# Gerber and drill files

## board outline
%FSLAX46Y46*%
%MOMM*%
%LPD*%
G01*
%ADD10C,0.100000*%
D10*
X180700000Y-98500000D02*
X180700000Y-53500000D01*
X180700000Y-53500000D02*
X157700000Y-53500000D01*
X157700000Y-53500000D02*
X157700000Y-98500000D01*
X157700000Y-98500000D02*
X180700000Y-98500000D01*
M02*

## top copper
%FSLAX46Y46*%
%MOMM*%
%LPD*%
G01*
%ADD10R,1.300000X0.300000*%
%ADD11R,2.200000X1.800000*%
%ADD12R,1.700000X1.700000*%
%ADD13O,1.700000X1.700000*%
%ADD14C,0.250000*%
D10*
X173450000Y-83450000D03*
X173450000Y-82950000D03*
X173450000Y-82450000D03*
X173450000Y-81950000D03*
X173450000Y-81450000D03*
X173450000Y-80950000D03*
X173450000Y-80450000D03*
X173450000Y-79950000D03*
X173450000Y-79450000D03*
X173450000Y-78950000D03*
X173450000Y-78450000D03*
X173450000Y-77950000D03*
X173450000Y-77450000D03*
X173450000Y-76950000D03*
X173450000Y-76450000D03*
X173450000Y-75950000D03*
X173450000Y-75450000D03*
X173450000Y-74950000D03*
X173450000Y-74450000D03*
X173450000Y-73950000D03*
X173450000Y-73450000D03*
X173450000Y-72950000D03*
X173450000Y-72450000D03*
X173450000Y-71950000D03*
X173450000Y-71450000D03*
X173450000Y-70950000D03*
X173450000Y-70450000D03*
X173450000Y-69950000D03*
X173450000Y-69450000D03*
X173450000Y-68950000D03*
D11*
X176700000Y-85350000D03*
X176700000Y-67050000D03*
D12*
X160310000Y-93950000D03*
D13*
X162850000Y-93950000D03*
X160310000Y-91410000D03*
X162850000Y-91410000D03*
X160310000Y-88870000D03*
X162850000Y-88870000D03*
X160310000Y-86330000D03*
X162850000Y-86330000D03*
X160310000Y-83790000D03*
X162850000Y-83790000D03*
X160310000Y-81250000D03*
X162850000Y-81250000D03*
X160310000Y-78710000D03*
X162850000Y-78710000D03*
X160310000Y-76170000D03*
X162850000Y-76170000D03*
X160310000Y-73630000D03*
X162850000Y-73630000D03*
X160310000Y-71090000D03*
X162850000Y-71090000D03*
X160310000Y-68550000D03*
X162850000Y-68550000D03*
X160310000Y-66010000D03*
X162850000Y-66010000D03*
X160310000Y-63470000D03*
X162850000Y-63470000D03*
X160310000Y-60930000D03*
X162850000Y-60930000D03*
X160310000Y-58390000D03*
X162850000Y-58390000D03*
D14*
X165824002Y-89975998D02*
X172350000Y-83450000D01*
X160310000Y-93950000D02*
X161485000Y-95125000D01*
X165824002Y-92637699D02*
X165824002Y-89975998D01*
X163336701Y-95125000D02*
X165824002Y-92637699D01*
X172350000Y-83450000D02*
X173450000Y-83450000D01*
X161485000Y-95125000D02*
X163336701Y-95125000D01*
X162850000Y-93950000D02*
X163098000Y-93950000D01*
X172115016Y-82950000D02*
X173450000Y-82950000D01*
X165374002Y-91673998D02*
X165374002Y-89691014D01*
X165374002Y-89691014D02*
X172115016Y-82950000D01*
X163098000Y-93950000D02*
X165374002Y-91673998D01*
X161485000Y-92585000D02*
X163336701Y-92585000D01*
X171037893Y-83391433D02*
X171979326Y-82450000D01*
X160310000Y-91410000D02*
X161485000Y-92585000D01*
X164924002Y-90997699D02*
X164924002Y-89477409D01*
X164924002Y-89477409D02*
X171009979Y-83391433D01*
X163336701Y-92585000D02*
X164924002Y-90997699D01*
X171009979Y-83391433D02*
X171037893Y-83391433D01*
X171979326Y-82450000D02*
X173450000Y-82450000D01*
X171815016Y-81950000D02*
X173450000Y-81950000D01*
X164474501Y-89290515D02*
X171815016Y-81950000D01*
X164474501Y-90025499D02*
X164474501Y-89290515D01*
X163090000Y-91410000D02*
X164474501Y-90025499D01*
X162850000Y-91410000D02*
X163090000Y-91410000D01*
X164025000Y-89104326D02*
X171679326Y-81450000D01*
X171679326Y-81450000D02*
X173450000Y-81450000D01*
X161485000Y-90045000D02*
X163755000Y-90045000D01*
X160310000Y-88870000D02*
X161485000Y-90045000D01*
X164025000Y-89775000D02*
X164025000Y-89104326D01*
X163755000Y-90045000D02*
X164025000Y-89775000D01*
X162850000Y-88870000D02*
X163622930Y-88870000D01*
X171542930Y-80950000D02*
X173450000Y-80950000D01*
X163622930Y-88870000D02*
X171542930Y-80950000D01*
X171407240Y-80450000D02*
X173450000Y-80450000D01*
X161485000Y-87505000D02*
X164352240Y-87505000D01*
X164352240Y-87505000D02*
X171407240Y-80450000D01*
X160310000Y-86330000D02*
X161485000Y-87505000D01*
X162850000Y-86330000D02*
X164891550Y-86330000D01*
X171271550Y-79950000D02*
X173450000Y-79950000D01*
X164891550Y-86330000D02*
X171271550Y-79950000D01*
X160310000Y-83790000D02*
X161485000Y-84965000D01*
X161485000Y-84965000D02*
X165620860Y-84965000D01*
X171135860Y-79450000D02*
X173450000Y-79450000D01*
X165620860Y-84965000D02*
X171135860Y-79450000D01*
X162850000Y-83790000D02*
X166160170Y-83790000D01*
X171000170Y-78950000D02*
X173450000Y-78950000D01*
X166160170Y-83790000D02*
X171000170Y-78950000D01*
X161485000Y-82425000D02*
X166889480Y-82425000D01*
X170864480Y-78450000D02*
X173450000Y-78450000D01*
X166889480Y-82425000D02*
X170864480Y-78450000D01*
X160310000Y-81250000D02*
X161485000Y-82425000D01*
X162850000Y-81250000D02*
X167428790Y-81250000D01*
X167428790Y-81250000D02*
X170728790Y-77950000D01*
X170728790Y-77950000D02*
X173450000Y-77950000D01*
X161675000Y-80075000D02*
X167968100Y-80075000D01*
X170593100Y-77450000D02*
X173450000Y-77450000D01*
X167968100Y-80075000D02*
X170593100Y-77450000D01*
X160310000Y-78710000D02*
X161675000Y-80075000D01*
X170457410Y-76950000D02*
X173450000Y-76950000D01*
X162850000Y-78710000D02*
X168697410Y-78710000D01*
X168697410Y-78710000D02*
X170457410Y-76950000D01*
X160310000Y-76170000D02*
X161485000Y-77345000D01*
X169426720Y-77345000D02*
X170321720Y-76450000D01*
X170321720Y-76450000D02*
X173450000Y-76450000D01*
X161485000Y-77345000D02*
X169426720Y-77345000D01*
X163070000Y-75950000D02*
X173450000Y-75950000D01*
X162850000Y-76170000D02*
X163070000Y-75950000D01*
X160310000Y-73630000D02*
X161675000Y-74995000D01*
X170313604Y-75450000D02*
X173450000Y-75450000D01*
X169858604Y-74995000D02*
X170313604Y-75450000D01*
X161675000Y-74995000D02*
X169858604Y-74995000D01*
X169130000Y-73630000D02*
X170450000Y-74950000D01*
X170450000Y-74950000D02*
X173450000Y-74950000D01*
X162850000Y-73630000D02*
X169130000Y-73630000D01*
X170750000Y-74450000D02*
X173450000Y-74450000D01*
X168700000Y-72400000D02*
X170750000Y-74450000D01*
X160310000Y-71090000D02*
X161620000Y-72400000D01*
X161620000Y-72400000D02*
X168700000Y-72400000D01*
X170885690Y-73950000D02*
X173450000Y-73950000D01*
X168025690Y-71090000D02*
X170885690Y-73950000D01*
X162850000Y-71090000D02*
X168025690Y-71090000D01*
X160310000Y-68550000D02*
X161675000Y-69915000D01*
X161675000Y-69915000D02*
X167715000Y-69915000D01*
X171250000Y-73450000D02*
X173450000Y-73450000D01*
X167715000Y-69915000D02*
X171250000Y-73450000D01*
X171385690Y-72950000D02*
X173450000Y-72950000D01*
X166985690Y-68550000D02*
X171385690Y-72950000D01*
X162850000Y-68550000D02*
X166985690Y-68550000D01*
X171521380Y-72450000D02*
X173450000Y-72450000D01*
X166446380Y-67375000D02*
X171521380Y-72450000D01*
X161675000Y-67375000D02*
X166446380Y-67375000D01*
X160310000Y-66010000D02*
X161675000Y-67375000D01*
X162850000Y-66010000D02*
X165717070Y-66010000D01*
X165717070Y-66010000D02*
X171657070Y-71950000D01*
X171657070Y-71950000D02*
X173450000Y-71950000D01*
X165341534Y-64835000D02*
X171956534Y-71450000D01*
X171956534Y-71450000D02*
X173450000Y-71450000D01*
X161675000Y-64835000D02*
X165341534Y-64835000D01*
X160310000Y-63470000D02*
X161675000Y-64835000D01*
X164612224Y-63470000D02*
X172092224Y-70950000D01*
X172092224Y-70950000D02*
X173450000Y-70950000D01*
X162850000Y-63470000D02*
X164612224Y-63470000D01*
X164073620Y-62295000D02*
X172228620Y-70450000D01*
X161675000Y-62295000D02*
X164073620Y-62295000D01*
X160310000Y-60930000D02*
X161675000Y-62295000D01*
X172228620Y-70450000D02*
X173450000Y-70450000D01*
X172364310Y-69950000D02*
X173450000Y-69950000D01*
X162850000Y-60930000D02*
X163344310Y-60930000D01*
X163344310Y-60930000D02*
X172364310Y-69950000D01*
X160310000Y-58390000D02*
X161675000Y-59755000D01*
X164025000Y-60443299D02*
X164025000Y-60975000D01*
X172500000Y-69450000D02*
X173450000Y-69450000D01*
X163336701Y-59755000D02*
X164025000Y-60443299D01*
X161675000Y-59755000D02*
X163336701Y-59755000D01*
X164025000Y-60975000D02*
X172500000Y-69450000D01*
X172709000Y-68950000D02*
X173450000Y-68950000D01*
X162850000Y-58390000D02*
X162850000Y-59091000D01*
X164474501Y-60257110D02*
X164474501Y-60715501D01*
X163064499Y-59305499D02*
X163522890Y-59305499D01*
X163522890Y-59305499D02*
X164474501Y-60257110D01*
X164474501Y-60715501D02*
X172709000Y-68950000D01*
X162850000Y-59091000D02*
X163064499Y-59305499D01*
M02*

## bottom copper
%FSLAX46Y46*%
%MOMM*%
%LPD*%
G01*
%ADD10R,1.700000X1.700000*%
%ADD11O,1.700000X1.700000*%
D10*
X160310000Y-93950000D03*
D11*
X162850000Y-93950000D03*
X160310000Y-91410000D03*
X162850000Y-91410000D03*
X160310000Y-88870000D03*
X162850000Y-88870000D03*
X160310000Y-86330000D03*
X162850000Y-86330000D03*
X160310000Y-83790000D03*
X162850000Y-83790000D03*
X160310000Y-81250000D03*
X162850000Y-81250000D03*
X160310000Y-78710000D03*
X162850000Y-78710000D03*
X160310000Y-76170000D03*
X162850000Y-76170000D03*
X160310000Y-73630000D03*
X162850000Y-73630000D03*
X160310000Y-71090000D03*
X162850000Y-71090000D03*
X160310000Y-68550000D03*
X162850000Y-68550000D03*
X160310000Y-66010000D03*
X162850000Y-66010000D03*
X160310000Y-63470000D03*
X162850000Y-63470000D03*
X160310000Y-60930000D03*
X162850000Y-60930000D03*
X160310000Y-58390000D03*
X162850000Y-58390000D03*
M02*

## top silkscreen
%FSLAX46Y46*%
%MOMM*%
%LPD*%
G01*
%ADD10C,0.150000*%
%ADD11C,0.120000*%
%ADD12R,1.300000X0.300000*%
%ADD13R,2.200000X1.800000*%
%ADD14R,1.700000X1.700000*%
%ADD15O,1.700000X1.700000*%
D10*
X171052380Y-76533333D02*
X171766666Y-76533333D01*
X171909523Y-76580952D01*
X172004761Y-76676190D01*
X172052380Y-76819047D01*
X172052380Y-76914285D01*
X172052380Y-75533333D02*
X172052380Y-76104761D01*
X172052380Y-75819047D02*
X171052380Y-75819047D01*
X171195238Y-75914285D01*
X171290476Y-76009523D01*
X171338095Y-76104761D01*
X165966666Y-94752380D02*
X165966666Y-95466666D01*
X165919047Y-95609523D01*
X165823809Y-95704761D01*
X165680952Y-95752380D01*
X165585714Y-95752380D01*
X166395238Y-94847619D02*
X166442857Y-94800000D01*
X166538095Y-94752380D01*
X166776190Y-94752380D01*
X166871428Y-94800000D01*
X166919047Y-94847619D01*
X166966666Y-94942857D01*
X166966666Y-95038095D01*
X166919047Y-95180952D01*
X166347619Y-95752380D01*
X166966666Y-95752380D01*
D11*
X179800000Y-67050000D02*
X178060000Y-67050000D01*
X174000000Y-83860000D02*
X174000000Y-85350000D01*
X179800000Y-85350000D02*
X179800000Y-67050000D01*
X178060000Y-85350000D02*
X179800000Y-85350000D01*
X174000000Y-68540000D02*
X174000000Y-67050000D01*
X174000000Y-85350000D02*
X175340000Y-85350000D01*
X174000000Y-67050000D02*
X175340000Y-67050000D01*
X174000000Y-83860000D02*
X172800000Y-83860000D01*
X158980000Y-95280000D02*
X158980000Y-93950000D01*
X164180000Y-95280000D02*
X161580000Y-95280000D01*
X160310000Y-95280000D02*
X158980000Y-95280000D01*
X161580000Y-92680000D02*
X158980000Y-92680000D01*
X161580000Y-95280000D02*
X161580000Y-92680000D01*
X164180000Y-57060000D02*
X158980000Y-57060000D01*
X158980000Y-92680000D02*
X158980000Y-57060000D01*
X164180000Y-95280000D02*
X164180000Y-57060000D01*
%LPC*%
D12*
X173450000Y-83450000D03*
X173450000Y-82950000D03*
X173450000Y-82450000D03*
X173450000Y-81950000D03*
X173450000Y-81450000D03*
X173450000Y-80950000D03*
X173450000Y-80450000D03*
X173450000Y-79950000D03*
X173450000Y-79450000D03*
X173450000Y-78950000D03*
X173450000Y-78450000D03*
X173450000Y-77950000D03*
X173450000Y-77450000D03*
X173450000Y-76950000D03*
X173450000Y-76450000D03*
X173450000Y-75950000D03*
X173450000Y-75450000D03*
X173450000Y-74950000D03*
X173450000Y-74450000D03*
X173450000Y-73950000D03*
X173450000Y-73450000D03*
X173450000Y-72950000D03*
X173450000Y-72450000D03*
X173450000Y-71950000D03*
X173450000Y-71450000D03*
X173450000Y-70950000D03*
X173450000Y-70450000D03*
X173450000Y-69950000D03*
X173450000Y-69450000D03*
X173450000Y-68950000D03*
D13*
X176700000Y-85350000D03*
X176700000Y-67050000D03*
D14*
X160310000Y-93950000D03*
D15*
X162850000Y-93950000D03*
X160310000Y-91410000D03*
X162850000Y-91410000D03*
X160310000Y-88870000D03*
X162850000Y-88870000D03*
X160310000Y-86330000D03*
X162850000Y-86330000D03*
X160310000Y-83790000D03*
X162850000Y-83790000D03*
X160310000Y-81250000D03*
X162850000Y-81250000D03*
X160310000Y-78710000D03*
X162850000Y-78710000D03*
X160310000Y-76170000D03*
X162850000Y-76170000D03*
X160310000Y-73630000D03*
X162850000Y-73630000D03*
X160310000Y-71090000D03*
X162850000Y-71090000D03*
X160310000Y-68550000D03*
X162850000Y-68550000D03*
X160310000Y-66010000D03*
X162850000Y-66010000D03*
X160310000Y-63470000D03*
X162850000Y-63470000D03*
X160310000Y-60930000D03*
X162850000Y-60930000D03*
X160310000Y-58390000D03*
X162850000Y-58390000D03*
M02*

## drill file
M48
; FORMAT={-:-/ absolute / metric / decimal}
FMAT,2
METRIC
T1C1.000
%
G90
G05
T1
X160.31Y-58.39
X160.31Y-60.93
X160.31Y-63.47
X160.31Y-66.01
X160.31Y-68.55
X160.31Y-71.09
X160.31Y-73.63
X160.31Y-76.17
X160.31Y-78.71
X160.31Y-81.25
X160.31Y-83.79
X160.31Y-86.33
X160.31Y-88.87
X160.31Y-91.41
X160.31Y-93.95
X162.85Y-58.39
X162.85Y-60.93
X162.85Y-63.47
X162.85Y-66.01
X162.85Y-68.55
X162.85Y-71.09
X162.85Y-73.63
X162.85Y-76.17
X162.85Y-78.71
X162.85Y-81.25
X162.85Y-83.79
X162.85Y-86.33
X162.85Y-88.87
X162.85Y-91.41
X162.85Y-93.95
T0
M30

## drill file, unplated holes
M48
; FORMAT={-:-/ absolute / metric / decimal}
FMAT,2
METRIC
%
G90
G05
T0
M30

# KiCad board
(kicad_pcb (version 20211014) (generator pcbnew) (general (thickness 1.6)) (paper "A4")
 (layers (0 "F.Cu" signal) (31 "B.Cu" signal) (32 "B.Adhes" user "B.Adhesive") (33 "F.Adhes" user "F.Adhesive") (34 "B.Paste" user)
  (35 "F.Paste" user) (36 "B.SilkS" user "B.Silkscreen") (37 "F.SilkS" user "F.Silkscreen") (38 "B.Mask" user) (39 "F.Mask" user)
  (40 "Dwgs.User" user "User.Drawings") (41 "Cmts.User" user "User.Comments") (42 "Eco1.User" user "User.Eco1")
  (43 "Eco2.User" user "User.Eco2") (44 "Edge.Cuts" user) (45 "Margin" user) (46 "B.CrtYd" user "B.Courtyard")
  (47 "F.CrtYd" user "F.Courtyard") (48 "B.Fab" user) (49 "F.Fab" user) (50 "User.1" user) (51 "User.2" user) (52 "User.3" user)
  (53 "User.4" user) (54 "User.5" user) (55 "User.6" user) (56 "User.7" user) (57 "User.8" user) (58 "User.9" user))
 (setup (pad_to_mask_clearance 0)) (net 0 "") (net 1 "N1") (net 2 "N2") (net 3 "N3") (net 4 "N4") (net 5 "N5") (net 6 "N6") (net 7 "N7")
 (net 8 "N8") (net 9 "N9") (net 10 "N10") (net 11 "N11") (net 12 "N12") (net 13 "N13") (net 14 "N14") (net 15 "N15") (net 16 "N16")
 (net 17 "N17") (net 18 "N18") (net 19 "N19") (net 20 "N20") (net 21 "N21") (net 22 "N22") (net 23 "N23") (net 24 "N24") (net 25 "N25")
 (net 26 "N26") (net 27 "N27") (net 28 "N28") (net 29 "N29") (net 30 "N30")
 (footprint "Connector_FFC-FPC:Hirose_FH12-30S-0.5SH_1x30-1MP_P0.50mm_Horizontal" (layer "F.Cu") (at 175.3 76.2 90)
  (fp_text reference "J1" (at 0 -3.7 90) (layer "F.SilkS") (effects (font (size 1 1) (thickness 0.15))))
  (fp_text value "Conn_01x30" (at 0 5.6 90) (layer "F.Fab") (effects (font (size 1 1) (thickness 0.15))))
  (fp_line (start 9.15 4.5) (end 9.15 2.76) (layer "F.SilkS") (width 0.12))
  (fp_line (start -7.66 -1.3) (end -9.15 -1.3) (layer "F.SilkS") (width 0.12))
  (fp_line (start -9.15 4.5) (end 9.15 4.5) (layer "F.SilkS") (width 0.12))
  (fp_line (start -9.15 2.76) (end -9.15 4.5) (layer "F.SilkS") (width 0.12))
  (fp_line (start 7.66 -1.3) (end 9.15 -1.3) (layer "F.SilkS") (width 0.12))
  (fp_line (start -9.15 -1.3) (end -9.15 0.04) (layer "F.SilkS") (width 0.12))
  (fp_line (start 9.15 -1.3) (end 9.15 0.04) (layer "F.SilkS") (width 0.12))
  (fp_line (start -7.66 -1.3) (end -7.66 -2.5) (layer "F.SilkS") (width 0.12))
  (pad "1" smd rect (at -7.25 -1.85 90) (size 0.3 1.3) (layers "F.Cu" "F.Paste" "F.Mask") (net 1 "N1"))
  (pad "2" smd rect (at -6.75 -1.85 90) (size 0.3 1.3) (layers "F.Cu" "F.Paste" "F.Mask") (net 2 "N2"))
  (pad "3" smd rect (at -6.25 -1.85 90) (size 0.3 1.3) (layers "F.Cu" "F.Paste" "F.Mask") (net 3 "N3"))
  (pad "4" smd rect (at -5.75 -1.85 90) (size 0.3 1.3) (layers "F.Cu" "F.Paste" "F.Mask") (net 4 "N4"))
  (pad "5" smd rect (at -5.25 -1.85 90) (size 0.3 1.3) (layers "F.Cu" "F.Paste" "F.Mask") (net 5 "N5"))
  (pad "6" smd rect (at -4.75 -1.85 90) (size 0.3 1.3) (layers "F.Cu" "F.Paste" "F.Mask") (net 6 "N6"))
  (pad "7" smd rect (at -4.25 -1.85 90) (size 0.3 1.3) (layers "F.Cu" "F.Paste" "F.Mask") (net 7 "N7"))
  (pad "8" smd rect (at -3.75 -1.85 90) (size 0.3 1.3) (layers "F.Cu" "F.Paste" "F.Mask") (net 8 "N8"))
  (pad "9" smd rect (at -3.25 -1.85 90) (size 0.3 1.3) (layers "F.Cu" "F.Paste" "F.Mask") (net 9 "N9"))
  (pad "10" smd rect (at -2.75 -1.85 90) (size 0.3 1.3) (layers "F.Cu" "F.Paste" "F.Mask") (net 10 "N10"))
  (pad "11" smd rect (at -2.25 -1.85 90) (size 0.3 1.3) (layers "F.Cu" "F.Paste" "F.Mask") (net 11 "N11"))
  (pad "12" smd rect (at -1.75 -1.85 90) (size 0.3 1.3) (layers "F.Cu" "F.Paste" "F.Mask") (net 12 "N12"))
  (pad "13" smd rect (at -1.25 -1.85 90) (size 0.3 1.3) (layers "F.Cu" "F.Paste" "F.Mask") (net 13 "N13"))
  (pad "14" smd rect (at -0.75 -1.85 90) (size 0.3 1.3) (layers "F.Cu" "F.Paste" "F.Mask") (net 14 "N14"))
  (pad "15" smd rect (at -0.25 -1.85 90) (size 0.3 1.3) (layers "F.Cu" "F.Paste" "F.Mask") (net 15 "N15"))
  (pad "16" smd rect (at 0.25 -1.85 90) (size 0.3 1.3) (layers "F.Cu" "F.Paste" "F.Mask") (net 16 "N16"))
  (pad "17" smd rect (at 0.75 -1.85 90) (size 0.3 1.3) (layers "F.Cu" "F.Paste" "F.Mask") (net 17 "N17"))
  (pad "18" smd rect (at 1.25 -1.85 90) (size 0.3 1.3) (layers "F.Cu" "F.Paste" "F.Mask") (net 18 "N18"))
  (pad "19" smd rect (at 1.75 -1.85 90) (size 0.3 1.3) (layers "F.Cu" "F.Paste" "F.Mask") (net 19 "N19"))
  (pad "20" smd rect (at 2.25 -1.85 90) (size 0.3 1.3) (layers "F.Cu" "F.Paste" "F.Mask") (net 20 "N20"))
  (pad "21" smd rect (at 2.75 -1.85 90) (size 0.3 1.3) (layers "F.Cu" "F.Paste" "F.Mask") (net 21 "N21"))
  (pad "22" smd rect (at 3.25 -1.85 90) (size 0.3 1.3) (layers "F.Cu" "F.Paste" "F.Mask") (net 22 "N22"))
  (pad "23" smd rect (at 3.75 -1.85 90) (size 0.3 1.3) (layers "F.Cu" "F.Paste" "F.Mask") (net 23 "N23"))
  (pad "24" smd rect (at 4.25 -1.85 90) (size 0.3 1.3) (layers "F.Cu" "F.Paste" "F.Mask") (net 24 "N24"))
  (pad "25" smd rect (at 4.75 -1.85 90) (size 0.3 1.3) (layers "F.Cu" "F.Paste" "F.Mask") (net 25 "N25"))
  (pad "26" smd rect (at 5.25 -1.85 90) (size 0.3 1.3) (layers "F.Cu" "F.Paste" "F.Mask") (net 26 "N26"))
  (pad "27" smd rect (at 5.75 -1.85 90) (size 0.3 1.3) (layers "F.Cu" "F.Paste" "F.Mask") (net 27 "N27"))
  (pad "28" smd rect (at 6.25 -1.85 90) (size 0.3 1.3) (layers "F.Cu" "F.Paste" "F.Mask") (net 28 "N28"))
  (pad "29" smd rect (at 6.75 -1.85 90) (size 0.3 1.3) (layers "F.Cu" "F.Paste" "F.Mask") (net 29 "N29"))
  (pad "30" smd rect (at 7.25 -1.85 90) (size 0.3 1.3) (layers "F.Cu" "F.Paste" "F.Mask") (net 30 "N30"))
  (pad "MP" smd rect (at -9.15 1.4 90) (size 1.8 2.2) (layers "F.Cu" "F.Paste" "F.Mask"))
  (pad "MP" smd rect (at 9.15 1.4 90) (size 1.8 2.2) (layers "F.Cu" "F.Paste" "F.Mask")))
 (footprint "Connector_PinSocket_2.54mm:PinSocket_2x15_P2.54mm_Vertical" (layer "F.Cu") (at 160.31 93.95 180)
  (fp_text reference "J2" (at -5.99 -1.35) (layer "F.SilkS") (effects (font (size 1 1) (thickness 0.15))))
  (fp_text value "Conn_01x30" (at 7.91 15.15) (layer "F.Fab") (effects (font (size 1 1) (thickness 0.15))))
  (fp_line (start 1.33 -1.33) (end 1.33 0) (layer "F.SilkS") (width 0.12))
  (fp_line (start -3.87 -1.33) (end -1.27 -1.33) (layer "F.SilkS") (width 0.12))
  (fp_line (start 0 -1.33) (end 1.33 -1.33) (layer "F.SilkS") (width 0.12))
  (fp_line (start -1.27 1.27) (end 1.33 1.27) (layer "F.SilkS") (width 0.12))
  (fp_line (start -1.27 -1.33) (end -1.27 1.27) (layer "F.SilkS") (width 0.12))
  (fp_line (start -3.87 36.89) (end 1.33 36.89) (layer "F.SilkS") (width 0.12))
  (fp_line (start 1.33 1.27) (end 1.33 36.89) (layer "F.SilkS") (width 0.12))
  (fp_line (start -3.87 -1.33) (end -3.87 36.89) (layer "F.SilkS") (width 0.12))
  (pad "1" thru_hole rect (at 0 0 180) (size 1.7 1.7) (drill 1) (layers *.Cu *.Mask) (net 1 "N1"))
  (pad "2" thru_hole oval (at -2.54 0 180) (size 1.7 1.7) (drill 1) (layers *.Cu *.Mask) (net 2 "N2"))
  (pad "3" thru_hole oval (at 0 2.54 180) (size 1.7 1.7) (drill 1) (layers *.Cu *.Mask) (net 3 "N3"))
  (pad "4" thru_hole oval (at -2.54 2.54 180) (size 1.7 1.7) (drill 1) (layers *.Cu *.Mask) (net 4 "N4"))
  (pad "5" thru_hole oval (at 0 5.08 180) (size 1.7 1.7) (drill 1) (layers *.Cu *.Mask) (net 5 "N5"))
  (pad "6" thru_hole oval (at -2.54 5.08 180) (size 1.7 1.7) (drill 1) (layers *.Cu *.Mask) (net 6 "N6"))
  (pad "7" thru_hole oval (at 0 7.62 180) (size 1.7 1.7) (drill 1) (layers *.Cu *.Mask) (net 7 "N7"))
  (pad "8" thru_hole oval (at -2.54 7.62 180) (size 1.7 1.7) (drill 1) (layers *.Cu *.Mask) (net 8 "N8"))
  (pad "9" thru_hole oval (at 0 10.16 180) (size 1.7 1.7) (drill 1) (layers *.Cu *.Mask) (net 9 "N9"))
  (pad "10" thru_hole oval (at -2.54 10.16 180) (size 1.7 1.7) (drill 1) (layers *.Cu *.Mask) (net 10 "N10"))
  (pad "11" thru_hole oval (at 0 12.7 180) (size 1.7 1.7) (drill 1) (layers *.Cu *.Mask) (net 11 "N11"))
  (pad "12" thru_hole oval (at -2.54 12.7 180) (size 1.7 1.7) (drill 1) (layers *.Cu *.Mask) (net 12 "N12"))
  (pad "13" thru_hole oval (at 0 15.24 180) (size 1.7 1.7) (drill 1) (layers *.Cu *.Mask) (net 13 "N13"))
  (pad "14" thru_hole oval (at -2.54 15.24 180) (size 1.7 1.7) (drill 1) (layers *.Cu *.Mask) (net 14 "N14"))
  (pad "15" thru_hole oval (at 0 17.78 180) (size 1.7 1.7) (drill 1) (layers *.Cu *.Mask) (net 15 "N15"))
  (pad "16" thru_hole oval (at -2.54 17.78 180) (size 1.7 1.7) (drill 1) (layers *.Cu *.Mask) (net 16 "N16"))
  (pad "17" thru_hole oval (at 0 20.32 180) (size 1.7 1.7) (drill 1) (layers *.Cu *.Mask) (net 17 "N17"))
  (pad "18" thru_hole oval (at -2.54 20.32 180) (size 1.7 1.7) (drill 1) (layers *.Cu *.Mask) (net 18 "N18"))
  (pad "19" thru_hole oval (at 0 22.86 180) (size 1.7 1.7) (drill 1) (layers *.Cu *.Mask) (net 19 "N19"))
  (pad "20" thru_hole oval (at -2.54 22.86 180) (size 1.7 1.7) (drill 1) (layers *.Cu *.Mask) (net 20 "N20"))
  (pad "21" thru_hole oval (at 0 25.4 180) (size 1.7 1.7) (drill 1) (layers *.Cu *.Mask) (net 21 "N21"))
  (pad "22" thru_hole oval (at -2.54 25.4 180) (size 1.7 1.7) (drill 1) (layers *.Cu *.Mask) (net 22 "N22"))
  (pad "23" thru_hole oval (at 0 27.94 180) (size 1.7 1.7) (drill 1) (layers *.Cu *.Mask) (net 23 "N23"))
  (pad "24" thru_hole oval (at -2.54 27.94 180) (size 1.7 1.7) (drill 1) (layers *.Cu *.Mask) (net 24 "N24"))
  (pad "25" thru_hole oval (at 0 30.48 180) (size 1.7 1.7) (drill 1) (layers *.Cu *.Mask) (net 25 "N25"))
  (pad "26" thru_hole oval (at -2.54 30.48 180) (size 1.7 1.7) (drill 1) (layers *.Cu *.Mask) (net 26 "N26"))
  (pad "27" thru_hole oval (at 0 33.02 180) (size 1.7 1.7) (drill 1) (layers *.Cu *.Mask) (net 27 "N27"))
  (pad "28" thru_hole oval (at -2.54 33.02 180) (size 1.7 1.7) (drill 1) (layers *.Cu *.Mask) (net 28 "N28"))
  (pad "29" thru_hole oval (at 0 35.56 180) (size 1.7 1.7) (drill 1) (layers *.Cu *.Mask) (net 29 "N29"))
  (pad "30" thru_hole oval (at -2.54 35.56 180) (size 1.7 1.7) (drill 1) (layers *.Cu *.Mask) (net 30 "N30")))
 (gr_line (start 180.7 98.5) (end 180.7 53.5) (layer "Edge.Cuts") (width 0.1))
 (gr_line (start 180.7 53.5) (end 157.7 53.5) (layer "Edge.Cuts") (width 0.1))
 (gr_line (start 157.7 53.5) (end 157.7 98.5) (layer "Edge.Cuts") (width 0.1))
 (gr_line (start 157.7 98.5) (end 180.7 98.5) (layer "Edge.Cuts") (width 0.1))
 (segment (start 165.824002 89.975998) (end 172.35 83.45) (width 0.25) (layer "F.Cu") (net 1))
 (segment (start 160.31 93.95) (end 161.485 95.125) (width 0.25) (layer "F.Cu") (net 1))
 (segment (start 165.824002 92.637699) (end 165.824002 89.975998) (width 0.25) (layer "F.Cu") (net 1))
 (segment (start 163.336701 95.125) (end 165.824002 92.637699) (width 0.25) (layer "F.Cu") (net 1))
 (segment (start 172.35 83.45) (end 173.45 83.45) (width 0.25) (layer "F.Cu") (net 1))
 (segment (start 161.485 95.125) (end 163.336701 95.125) (width 0.25) (layer "F.Cu") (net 1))
 (segment (start 162.85 93.95) (end 163.098 93.95) (width 0.25) (layer "F.Cu") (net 2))
 (segment (start 172.115016 82.95) (end 173.45 82.95) (width 0.25) (layer "F.Cu") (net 2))
 (segment (start 165.374002 91.673998) (end 165.374002 89.691014) (width 0.25) (layer "F.Cu") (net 2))
 (segment (start 165.374002 89.691014) (end 172.115016 82.95) (width 0.25) (layer "F.Cu") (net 2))
 (segment (start 163.098 93.95) (end 165.374002 91.673998) (width 0.25) (layer "F.Cu") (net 2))
 (segment (start 161.485 92.585) (end 163.336701 92.585) (width 0.25) (layer "F.Cu") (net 3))
 (segment (start 171.037893 83.391433) (end 171.979326 82.45) (width 0.25) (layer "F.Cu") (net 3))
 (segment (start 160.31 91.41) (end 161.485 92.585) (width 0.25) (layer "F.Cu") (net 3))
 (segment (start 164.924002 90.997699) (end 164.924002 89.477409) (width 0.25) (layer "F.Cu") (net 3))
 (segment (start 164.924002 89.477409) (end 171.009979 83.391433) (width 0.25) (layer "F.Cu") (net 3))
 (segment (start 163.336701 92.585) (end 164.924002 90.997699) (width 0.25) (layer "F.Cu") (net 3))
 (segment (start 171.009979 83.391433) (end 171.037893 83.391433) (width 0.25) (layer "F.Cu") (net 3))
 (segment (start 171.979326 82.45) (end 173.45 82.45) (width 0.25) (layer "F.Cu") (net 3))
 (segment (start 171.815016 81.95) (end 173.45 81.95) (width 0.25) (layer "F.Cu") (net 4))
 (segment (start 164.474501 89.290515) (end 171.815016 81.95) (width 0.25) (layer "F.Cu") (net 4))
 (segment (start 164.474501 90.025499) (end 164.474501 89.290515) (width 0.25) (layer "F.Cu") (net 4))
 (segment (start 163.09 91.41) (end 164.474501 90.025499) (width 0.25) (layer "F.Cu") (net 4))
 (segment (start 162.85 91.41) (end 163.09 91.41) (width 0.25) (layer "F.Cu") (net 4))
 (segment (start 164.025 89.104326) (end 171.679326 81.45) (width 0.25) (layer "F.Cu") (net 5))
 (segment (start 171.679326 81.45) (end 173.45 81.45) (width 0.25) (layer "F.Cu") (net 5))
 (segment (start 161.485 90.045) (end 163.755 90.045) (width 0.25) (layer "F.Cu") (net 5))
 (segment (start 160.31 88.87) (end 161.485 90.045) (width 0.25) (layer "F.Cu") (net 5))
 (segment (start 164.025 89.775) (end 164.025 89.104326) (width 0.25) (layer "F.Cu") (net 5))
 (segment (start 163.755 90.045) (end 164.025 89.775) (width 0.25) (layer "F.Cu") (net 5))
 (segment (start 162.85 88.87) (end 163.62293 88.87) (width 0.25) (layer "F.Cu") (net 6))
 (segment (start 171.54293 80.95) (end 173.45 80.95) (width 0.25) (layer "F.Cu") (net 6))
 (segment (start 163.62293 88.87) (end 171.54293 80.95) (width 0.25) (layer "F.Cu") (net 6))
 (segment (start 171.40724 80.45) (end 173.45 80.45) (width 0.25) (layer "F.Cu") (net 7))
 (segment (start 161.485 87.505) (end 164.35224 87.505) (width 0.25) (layer "F.Cu") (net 7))
 (segment (start 164.35224 87.505) (end 171.40724 80.45) (width 0.25) (layer "F.Cu") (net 7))
 (segment (start 160.31 86.33) (end 161.485 87.505) (width 0.25) (layer "F.Cu") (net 7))
 (segment (start 162.85 86.33) (end 164.89155 86.33) (width 0.25) (layer "F.Cu") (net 8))
 (segment (start 171.27155 79.95) (end 173.45 79.95) (width 0.25) (layer "F.Cu") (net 8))
 (segment (start 164.89155 86.33) (end 171.27155 79.95) (width 0.25) (layer "F.Cu") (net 8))
 (segment (start 160.31 83.79) (end 161.485 84.965) (width 0.25) (layer "F.Cu") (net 9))
 (segment (start 161.485 84.965) (end 165.62086 84.965) (width 0.25) (layer "F.Cu") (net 9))
 (segment (start 171.13586 79.45) (end 173.45 79.45) (width 0.25) (layer "F.Cu") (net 9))
 (segment (start 165.62086 84.965) (end 171.13586 79.45) (width 0.25) (layer "F.Cu") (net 9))
 (segment (start 162.85 83.79) (end 166.16017 83.79) (width 0.25) (layer "F.Cu") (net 10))
 (segment (start 171.00017 78.95) (end 173.45 78.95) (width 0.25) (layer "F.Cu") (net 10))
 (segment (start 166.16017 83.79) (end 171.00017 78.95) (width 0.25) (layer "F.Cu") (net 10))
 (segment (start 161.485 82.425) (end 166.88948 82.425) (width 0.25) (layer "F.Cu") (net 11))
 (segment (start 170.86448 78.45) (end 173.45 78.45) (width 0.25) (layer "F.Cu") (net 11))
 (segment (start 166.88948 82.425) (end 170.86448 78.45) (width 0.25) (layer "F.Cu") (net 11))
 (segment (start 160.31 81.25) (end 161.485 82.425) (width 0.25) (layer "F.Cu") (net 11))
 (segment (start 162.85 81.25) (end 167.42879 81.25) (width 0.25) (layer "F.Cu") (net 12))
 (segment (start 167.42879 81.25) (end 170.72879 77.95) (width 0.25) (layer "F.Cu") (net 12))
 (segment (start 170.72879 77.95) (end 173.45 77.95) (width 0.25) (layer "F.Cu") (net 12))
 (segment (start 161.675 80.075) (end 167.9681 80.075) (width 0.25) (layer "F.Cu") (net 13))
 (segment (start 170.5931 77.45) (end 173.45 77.45) (width 0.25) (layer "F.Cu") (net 13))
 (segment (start 167.9681 80.075) (end 170.5931 77.45) (width 0.25) (layer "F.Cu") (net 13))
 (segment (start 160.31 78.71) (end 161.675 80.075) (width 0.25) (layer "F.Cu") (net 13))
 (segment (start 170.45741 76.95) (end 173.45 76.95) (width 0.25) (layer "F.Cu") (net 14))
 (segment (start 162.85 78.71) (end 168.69741 78.71) (width 0.25) (layer "F.Cu") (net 14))
 (segment (start 168.69741 78.71) (end 170.45741 76.95) (width 0.25) (layer "F.Cu") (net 14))
 (segment (start 160.31 76.17) (end 161.485 77.345) (width 0.25) (layer "F.Cu") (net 15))
 (segment (start 169.42672 77.345) (end 170.32172 76.45) (width 0.25) (layer "F.Cu") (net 15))
 (segment (start 170.32172 76.45) (end 173.45 76.45) (width 0.25) (layer "F.Cu") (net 15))
 (segment (start 161.485 77.345) (end 169.42672 77.345) (width 0.25) (layer "F.Cu") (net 15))
 (segment (start 163.07 75.95) (end 173.45 75.95) (width 0.25) (layer "F.Cu") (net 16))
 (segment (start 162.85 76.17) (end 163.07 75.95) (width 0.25) (layer "F.Cu") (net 16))
 (segment (start 160.31 73.63) (end 161.675 74.995) (width 0.25) (layer "F.Cu") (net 17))
 (segment (start 170.313604 75.45) (end 173.45 75.45) (width 0.25) (layer "F.Cu") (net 17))
 (segment (start 169.858604 74.995) (end 170.313604 75.45) (width 0.25) (layer "F.Cu") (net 17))
 (segment (start 161.675 74.995) (end 169.858604 74.995) (width 0.25) (layer "F.Cu") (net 17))
 (segment (start 169.13 73.63) (end 170.45 74.95) (width 0.25) (layer "F.Cu") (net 18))
 (segment (start 170.45 74.95) (end 173.45 74.95) (width 0.25) (layer "F.Cu") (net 18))
 (segment (start 162.85 73.63) (end 169.13 73.63) (width 0.25) (layer "F.Cu") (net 18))
 (segment (start 170.75 74.45) (end 173.45 74.45) (width 0.25) (layer "F.Cu") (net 19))
 (segment (start 168.7 72.4) (end 170.75 74.45) (width 0.25) (layer "F.Cu") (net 19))
 (segment (start 160.31 71.09) (end 161.62 72.4) (width 0.25) (layer "F.Cu") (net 19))
 (segment (start 161.62 72.4) (end 168.7 72.4) (width 0.25) (layer "F.Cu") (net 19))
 (segment (start 170.88569 73.95) (end 173.45 73.95) (width 0.25) (layer "F.Cu") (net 20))
 (segment (start 168.02569 71.09) (end 170.88569 73.95) (width 0.25) (layer "F.Cu") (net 20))
 (segment (start 162.85 71.09) (end 168.02569 71.09) (width 0.25) (layer "F.Cu") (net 20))
 (segment (start 160.31 68.55) (end 161.675 69.915) (width 0.25) (layer "F.Cu") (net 21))
 (segment (start 161.675 69.915) (end 167.715 69.915) (width 0.25) (layer "F.Cu") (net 21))
 (segment (start 171.25 73.45) (end 173.45 73.45) (width 0.25) (layer "F.Cu") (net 21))
 (segment (start 167.715 69.915) (end 171.25 73.45) (width 0.25) (layer "F.Cu") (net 21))
 (segment (start 171.38569 72.95) (end 173.45 72.95) (width 0.25) (layer "F.Cu") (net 22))
 (segment (start 166.98569 68.55) (end 171.38569 72.95) (width 0.25) (layer "F.Cu") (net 22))
 (segment (start 162.85 68.55) (end 166.98569 68.55) (width 0.25) (layer "F.Cu") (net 22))
 (segment (start 171.52138 72.45) (end 173.45 72.45) (width 0.25) (layer "F.Cu") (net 23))
 (segment (start 166.44638 67.375) (end 171.52138 72.45) (width 0.25) (layer "F.Cu") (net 23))
 (segment (start 161.675 67.375) (end 166.44638 67.375) (width 0.25) (layer "F.Cu") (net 23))
 (segment (start 160.31 66.01) (end 161.675 67.375) (width 0.25) (layer "F.Cu") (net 23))
 (segment (start 162.85 66.01) (end 165.71707 66.01) (width 0.25) (layer "F.Cu") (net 24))
 (segment (start 165.71707 66.01) (end 171.65707 71.95) (width 0.25) (layer "F.Cu") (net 24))
 (segment (start 171.65707 71.95) (end 173.45 71.95) (width 0.25) (layer "F.Cu") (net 24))
 (segment (start 165.341534 64.835) (end 171.956534 71.45) (width 0.25) (layer "F.Cu") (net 25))
 (segment (start 171.956534 71.45) (end 173.45 71.45) (width 0.25) (layer "F.Cu") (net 25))
 (segment (start 161.675 64.835) (end 165.341534 64.835) (width 0.25) (layer "F.Cu") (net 25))
 (segment (start 160.31 63.47) (end 161.675 64.835) (width 0.25) (layer "F.Cu") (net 25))
 (segment (start 164.612224 63.47) (end 172.092224 70.95) (width 0.25) (layer "F.Cu") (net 26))
 (segment (start 172.092224 70.95) (end 173.45 70.95) (width 0.25) (layer "F.Cu") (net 26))
 (segment (start 162.85 63.47) (end 164.612224 63.47) (width 0.25) (layer "F.Cu") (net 26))
 (segment (start 164.07362 62.295) (end 172.22862 70.45) (width 0.25) (layer "F.Cu") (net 27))
 (segment (start 161.675 62.295) (end 164.07362 62.295) (width 0.25) (layer "F.Cu") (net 27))
 (segment (start 160.31 60.93) (end 161.675 62.295) (width 0.25) (layer "F.Cu") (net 27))
 (segment (start 172.22862 70.45) (end 173.45 70.45) (width 0.25) (layer "F.Cu") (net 27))
 (segment (start 172.36431 69.95) (end 173.45 69.95) (width 0.25) (layer "F.Cu") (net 28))
 (segment (start 162.85 60.93) (end 163.34431 60.93) (width 0.25) (layer "F.Cu") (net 28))
 (segment (start 163.34431 60.93) (end 172.36431 69.95) (width 0.25) (layer "F.Cu") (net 28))
 (segment (start 160.31 58.39) (end 161.675 59.755) (width 0.25) (layer "F.Cu") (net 29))
 (segment (start 164.025 60.443299) (end 164.025 60.975) (width 0.25) (layer "F.Cu") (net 29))
 (segment (start 172.5 69.45) (end 173.45 69.45) (width 0.25) (layer "F.Cu") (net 29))
 (segment (start 163.336701 59.755) (end 164.025 60.443299) (width 0.25) (layer "F.Cu") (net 29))
 (segment (start 161.675 59.755) (end 163.336701 59.755) (width 0.25) (layer "F.Cu") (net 29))
 (segment (start 164.025 60.975) (end 172.5 69.45) (width 0.25) (layer "F.Cu") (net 29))
 (segment (start 172.709 68.95) (end 173.45 68.95) (width 0.25) (layer "F.Cu") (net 30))
 (segment (start 162.85 58.39) (end 162.85 59.091) (width 0.25) (layer "F.Cu") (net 30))
 (segment (start 164.474501 60.25711) (end 164.474501 60.715501) (width 0.25) (layer "F.Cu") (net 30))
 (segment (start 163.064499 59.305499) (end 163.52289 59.305499) (width 0.25) (layer "F.Cu") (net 30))
 (segment (start 163.52289 59.305499) (end 164.474501 60.25711) (width 0.25) (layer "F.Cu") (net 30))
 (segment (start 164.474501 60.715501) (end 172.709 68.95) (width 0.25) (layer "F.Cu") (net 30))
 (segment (start 162.85 59.091) (end 163.064499 59.305499) (width 0.25) (layer "F.Cu") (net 30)))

